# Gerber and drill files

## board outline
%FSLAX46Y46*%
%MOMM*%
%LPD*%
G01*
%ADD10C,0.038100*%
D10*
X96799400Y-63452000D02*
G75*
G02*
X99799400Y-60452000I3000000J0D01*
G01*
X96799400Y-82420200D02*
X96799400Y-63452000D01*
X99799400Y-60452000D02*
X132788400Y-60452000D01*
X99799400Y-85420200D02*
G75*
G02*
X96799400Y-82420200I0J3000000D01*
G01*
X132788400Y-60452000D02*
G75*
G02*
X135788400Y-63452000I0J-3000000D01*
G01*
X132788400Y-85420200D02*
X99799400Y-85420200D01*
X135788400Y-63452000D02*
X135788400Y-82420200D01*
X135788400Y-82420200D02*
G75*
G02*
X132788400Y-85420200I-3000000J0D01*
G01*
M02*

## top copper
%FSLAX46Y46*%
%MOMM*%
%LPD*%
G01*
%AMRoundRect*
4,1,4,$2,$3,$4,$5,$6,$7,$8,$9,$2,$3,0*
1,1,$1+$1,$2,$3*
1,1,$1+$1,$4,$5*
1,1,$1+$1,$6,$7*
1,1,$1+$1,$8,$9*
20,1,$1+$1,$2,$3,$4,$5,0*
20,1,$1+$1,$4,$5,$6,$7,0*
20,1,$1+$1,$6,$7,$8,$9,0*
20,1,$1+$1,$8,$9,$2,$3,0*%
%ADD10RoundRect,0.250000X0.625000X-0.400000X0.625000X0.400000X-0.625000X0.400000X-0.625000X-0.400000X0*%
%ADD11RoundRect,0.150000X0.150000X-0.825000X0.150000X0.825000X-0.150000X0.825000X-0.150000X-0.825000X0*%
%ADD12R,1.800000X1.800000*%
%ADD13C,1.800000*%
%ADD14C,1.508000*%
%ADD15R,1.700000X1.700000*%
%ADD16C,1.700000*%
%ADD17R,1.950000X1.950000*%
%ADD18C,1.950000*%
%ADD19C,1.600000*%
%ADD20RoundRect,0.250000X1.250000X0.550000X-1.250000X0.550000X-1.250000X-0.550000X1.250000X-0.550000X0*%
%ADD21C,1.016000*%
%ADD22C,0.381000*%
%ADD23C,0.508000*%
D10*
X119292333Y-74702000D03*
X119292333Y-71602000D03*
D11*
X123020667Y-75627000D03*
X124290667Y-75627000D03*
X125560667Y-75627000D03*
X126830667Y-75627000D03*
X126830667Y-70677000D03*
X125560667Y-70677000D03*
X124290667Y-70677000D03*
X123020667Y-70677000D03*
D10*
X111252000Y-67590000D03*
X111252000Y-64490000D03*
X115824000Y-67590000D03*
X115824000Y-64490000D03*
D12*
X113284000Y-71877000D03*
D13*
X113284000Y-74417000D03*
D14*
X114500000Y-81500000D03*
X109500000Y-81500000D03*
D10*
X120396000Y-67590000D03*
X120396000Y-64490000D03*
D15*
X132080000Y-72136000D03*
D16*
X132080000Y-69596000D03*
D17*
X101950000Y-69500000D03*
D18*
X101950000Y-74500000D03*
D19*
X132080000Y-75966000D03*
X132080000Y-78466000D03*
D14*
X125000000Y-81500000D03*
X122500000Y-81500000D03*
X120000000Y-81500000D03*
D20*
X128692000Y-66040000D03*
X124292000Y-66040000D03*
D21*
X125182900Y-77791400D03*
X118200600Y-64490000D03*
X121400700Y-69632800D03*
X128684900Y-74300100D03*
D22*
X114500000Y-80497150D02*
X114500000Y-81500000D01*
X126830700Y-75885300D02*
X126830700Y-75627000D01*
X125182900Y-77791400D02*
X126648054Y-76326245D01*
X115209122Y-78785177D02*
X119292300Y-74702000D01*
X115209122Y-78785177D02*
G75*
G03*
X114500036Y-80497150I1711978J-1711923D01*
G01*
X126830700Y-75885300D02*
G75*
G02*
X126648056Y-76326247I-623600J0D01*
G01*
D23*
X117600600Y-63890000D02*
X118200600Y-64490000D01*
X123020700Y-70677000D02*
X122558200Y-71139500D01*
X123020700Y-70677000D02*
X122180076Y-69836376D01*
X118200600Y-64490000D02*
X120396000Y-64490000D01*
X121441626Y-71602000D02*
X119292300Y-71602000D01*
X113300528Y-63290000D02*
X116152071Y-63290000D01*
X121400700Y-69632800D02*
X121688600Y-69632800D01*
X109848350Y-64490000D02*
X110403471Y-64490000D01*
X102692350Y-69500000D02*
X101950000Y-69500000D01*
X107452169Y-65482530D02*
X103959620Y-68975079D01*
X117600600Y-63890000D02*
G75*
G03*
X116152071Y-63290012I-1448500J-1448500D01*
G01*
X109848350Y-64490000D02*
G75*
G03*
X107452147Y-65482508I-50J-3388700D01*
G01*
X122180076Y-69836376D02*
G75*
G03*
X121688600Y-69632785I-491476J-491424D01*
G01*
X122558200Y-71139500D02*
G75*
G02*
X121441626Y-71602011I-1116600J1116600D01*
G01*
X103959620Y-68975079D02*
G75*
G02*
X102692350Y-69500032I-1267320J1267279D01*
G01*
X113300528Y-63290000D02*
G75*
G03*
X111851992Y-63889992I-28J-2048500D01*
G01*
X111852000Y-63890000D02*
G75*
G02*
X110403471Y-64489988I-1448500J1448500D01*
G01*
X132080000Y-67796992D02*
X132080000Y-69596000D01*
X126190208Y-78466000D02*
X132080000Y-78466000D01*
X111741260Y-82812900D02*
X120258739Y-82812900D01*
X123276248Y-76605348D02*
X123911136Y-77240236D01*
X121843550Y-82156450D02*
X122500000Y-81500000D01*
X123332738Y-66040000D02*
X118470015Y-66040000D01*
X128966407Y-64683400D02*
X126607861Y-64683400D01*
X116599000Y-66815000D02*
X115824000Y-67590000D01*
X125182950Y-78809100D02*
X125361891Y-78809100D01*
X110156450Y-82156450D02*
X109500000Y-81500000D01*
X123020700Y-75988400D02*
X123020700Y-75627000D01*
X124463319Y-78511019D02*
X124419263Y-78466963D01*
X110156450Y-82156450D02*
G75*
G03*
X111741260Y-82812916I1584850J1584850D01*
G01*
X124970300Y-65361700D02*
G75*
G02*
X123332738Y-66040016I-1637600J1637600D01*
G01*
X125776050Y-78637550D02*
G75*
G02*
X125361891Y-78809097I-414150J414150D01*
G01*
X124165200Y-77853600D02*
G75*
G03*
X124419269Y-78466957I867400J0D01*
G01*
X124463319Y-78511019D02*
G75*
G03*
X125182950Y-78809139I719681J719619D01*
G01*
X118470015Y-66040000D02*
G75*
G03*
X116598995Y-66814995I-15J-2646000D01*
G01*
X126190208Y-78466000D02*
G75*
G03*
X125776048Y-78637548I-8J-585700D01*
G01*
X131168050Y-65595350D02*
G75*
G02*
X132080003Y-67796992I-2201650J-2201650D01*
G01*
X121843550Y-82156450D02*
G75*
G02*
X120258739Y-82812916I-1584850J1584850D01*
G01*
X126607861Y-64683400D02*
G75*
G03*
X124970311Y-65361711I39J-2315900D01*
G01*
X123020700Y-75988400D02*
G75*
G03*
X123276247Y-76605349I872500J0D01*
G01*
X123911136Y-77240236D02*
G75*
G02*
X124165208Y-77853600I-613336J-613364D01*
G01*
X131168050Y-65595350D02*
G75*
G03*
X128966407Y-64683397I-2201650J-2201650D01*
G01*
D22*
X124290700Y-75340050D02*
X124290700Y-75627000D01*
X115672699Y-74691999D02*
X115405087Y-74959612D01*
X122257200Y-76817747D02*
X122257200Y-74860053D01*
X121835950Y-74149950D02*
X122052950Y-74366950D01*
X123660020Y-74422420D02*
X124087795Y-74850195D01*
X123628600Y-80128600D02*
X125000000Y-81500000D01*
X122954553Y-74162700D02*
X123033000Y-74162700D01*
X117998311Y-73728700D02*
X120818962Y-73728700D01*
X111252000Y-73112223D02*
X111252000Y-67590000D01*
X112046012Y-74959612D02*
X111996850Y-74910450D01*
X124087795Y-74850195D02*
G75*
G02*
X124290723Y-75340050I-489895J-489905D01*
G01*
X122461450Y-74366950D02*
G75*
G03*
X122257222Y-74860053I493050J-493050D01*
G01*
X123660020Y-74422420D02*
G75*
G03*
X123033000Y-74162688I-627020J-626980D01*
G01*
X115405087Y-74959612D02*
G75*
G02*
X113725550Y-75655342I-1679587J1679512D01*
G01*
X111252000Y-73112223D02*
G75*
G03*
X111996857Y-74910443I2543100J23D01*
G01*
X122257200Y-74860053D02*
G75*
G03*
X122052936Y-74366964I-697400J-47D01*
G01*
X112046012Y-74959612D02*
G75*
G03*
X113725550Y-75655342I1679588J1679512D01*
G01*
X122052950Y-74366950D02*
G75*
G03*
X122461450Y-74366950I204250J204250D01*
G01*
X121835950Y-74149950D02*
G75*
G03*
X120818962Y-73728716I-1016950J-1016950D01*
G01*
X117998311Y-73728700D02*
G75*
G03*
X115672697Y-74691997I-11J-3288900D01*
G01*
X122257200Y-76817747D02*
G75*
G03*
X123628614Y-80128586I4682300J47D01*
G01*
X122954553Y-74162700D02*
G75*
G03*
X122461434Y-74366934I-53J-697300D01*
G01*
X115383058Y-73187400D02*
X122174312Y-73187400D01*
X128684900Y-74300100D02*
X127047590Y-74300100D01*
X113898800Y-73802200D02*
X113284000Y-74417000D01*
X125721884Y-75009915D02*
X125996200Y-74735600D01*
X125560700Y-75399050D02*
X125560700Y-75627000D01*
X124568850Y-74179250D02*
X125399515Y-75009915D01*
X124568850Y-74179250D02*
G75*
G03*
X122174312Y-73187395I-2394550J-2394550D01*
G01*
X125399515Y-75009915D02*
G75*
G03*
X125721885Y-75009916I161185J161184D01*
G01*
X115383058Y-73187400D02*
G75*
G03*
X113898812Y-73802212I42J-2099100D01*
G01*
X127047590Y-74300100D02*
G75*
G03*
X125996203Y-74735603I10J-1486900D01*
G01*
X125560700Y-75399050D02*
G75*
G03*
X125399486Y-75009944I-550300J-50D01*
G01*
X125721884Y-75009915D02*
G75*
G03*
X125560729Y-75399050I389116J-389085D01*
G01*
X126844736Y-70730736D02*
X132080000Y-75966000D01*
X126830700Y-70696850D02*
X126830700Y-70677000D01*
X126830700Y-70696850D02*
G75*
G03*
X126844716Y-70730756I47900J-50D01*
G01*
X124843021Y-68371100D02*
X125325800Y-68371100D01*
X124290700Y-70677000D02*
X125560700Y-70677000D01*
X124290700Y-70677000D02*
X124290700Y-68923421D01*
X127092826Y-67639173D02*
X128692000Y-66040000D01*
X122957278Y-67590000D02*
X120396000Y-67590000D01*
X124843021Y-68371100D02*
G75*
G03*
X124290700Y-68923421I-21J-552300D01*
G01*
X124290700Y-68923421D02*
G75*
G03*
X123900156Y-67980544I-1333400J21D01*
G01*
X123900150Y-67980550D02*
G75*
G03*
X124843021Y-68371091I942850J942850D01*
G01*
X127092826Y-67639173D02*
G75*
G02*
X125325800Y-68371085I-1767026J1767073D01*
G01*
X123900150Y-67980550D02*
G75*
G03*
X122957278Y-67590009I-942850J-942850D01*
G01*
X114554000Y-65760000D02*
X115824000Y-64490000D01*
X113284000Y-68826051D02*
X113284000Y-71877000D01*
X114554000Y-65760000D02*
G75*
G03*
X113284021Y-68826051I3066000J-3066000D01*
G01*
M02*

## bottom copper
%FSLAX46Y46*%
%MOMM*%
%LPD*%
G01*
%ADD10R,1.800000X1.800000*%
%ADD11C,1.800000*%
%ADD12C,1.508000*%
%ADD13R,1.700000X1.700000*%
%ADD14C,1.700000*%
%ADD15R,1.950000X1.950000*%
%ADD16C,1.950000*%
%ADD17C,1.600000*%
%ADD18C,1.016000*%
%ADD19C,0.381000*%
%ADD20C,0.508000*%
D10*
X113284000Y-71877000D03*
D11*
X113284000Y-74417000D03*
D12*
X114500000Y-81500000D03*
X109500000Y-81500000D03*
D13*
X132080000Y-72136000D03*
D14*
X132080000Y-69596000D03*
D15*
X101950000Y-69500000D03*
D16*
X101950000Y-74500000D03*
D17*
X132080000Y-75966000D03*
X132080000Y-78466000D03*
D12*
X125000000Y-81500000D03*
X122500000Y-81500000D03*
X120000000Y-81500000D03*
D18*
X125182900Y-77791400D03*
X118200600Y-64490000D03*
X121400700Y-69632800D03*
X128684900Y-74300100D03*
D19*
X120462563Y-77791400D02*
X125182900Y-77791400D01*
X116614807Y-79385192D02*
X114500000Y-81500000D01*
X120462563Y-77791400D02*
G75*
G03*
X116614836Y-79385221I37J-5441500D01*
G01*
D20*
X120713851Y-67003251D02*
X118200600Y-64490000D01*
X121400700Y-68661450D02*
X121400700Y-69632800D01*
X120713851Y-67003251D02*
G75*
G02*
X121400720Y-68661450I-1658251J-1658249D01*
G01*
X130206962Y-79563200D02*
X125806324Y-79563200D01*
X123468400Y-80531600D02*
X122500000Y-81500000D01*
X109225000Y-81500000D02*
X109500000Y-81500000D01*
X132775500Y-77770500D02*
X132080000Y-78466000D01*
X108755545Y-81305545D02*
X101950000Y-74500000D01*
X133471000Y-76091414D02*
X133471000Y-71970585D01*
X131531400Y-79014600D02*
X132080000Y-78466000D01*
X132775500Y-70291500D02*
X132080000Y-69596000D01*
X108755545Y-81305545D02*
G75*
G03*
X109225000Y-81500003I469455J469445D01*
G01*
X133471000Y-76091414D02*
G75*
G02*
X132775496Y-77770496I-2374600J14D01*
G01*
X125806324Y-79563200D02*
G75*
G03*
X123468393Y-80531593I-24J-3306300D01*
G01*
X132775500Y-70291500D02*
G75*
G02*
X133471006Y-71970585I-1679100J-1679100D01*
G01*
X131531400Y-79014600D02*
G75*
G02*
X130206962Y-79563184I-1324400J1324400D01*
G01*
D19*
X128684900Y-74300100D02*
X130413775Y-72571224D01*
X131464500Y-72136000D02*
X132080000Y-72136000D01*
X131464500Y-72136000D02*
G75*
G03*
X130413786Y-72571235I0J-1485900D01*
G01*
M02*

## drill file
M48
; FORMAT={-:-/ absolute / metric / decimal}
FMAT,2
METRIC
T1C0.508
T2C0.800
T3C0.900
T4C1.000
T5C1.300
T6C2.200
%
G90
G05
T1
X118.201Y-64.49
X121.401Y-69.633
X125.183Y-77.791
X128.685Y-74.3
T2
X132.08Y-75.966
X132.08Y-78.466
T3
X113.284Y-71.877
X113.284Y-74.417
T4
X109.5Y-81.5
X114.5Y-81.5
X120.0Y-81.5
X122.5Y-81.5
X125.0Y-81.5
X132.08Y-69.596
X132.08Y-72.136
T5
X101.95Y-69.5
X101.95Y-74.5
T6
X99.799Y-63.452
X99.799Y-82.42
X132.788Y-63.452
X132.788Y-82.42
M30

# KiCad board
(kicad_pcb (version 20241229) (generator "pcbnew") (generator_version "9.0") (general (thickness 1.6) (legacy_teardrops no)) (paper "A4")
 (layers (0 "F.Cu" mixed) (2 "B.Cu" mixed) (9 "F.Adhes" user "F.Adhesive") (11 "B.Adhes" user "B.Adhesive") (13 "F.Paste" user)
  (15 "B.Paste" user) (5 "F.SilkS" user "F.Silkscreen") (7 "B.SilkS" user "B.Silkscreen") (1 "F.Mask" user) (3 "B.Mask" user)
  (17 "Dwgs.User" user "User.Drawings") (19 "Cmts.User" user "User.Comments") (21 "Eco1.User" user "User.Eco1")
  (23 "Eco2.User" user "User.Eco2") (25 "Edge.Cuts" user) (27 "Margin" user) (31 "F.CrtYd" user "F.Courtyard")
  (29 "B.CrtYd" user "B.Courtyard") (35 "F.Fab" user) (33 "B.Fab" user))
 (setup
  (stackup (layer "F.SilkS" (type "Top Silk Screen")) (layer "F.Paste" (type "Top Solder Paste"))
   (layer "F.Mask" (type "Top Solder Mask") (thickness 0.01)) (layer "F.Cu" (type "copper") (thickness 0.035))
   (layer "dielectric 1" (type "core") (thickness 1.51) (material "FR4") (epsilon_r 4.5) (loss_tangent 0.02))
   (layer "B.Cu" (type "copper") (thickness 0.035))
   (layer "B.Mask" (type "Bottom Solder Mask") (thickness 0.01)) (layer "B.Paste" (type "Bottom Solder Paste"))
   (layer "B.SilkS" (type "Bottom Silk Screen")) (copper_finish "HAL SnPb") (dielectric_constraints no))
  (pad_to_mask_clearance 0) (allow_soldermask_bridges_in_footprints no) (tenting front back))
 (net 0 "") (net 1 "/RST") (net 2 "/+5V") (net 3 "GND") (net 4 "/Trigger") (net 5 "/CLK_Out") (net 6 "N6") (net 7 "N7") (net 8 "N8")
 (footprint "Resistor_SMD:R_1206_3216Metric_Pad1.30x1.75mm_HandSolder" (layer "F.Cu") (at 119.292333 73.152 90)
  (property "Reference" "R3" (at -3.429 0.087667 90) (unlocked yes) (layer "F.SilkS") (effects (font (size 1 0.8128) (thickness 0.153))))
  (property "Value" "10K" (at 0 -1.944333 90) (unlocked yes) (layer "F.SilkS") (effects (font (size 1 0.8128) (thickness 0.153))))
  (pad "1" smd roundrect (at -1.55 0 90) (size 1.3 1.75) (layers "F.Cu" "F.Mask" "F.Paste") (roundrect_rratio 0.192308) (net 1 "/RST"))
  (pad "2" smd roundrect (at 1.55 0 90) (size 1.3 1.75) (layers "F.Cu" "F.Mask" "F.Paste") (roundrect_rratio 0.192308) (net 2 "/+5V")))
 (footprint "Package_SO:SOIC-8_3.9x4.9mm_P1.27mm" (layer "F.Cu") (at 124.925667 73.152 90)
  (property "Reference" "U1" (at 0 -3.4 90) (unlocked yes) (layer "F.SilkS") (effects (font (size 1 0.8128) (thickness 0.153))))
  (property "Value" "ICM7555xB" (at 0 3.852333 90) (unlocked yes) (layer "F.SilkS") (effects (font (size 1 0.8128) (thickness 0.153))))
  (pad "1" smd roundrect (at -2.475 -1.905 90) (size 1.95 0.6) (layers "F.Cu" "F.Mask" "F.Paste") (roundrect_rratio 0.25) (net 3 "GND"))
  (pad "2" smd roundrect (at -2.475 -0.635 90) (size 1.95 0.6) (layers "F.Cu" "F.Mask" "F.Paste") (roundrect_rratio 0.25) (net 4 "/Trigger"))
  (pad "3" smd roundrect (at -2.475 0.635 90) (size 1.95 0.6) (layers "F.Cu" "F.Mask" "F.Paste") (roundrect_rratio 0.25) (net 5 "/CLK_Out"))
  (pad "4" smd roundrect (at -2.475 1.905 90) (size 1.95 0.6) (layers "F.Cu" "F.Mask" "F.Paste") (roundrect_rratio 0.25) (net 1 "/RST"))
  (pad "5" smd roundrect (at 2.475 1.905 90) (size 1.95 0.6) (layers "F.Cu" "F.Mask" "F.Paste") (roundrect_rratio 0.25) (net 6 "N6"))
  (pad "6" smd roundrect (at 2.475 0.635 90) (size 1.95 0.6) (layers "F.Cu" "F.Mask" "F.Paste") (roundrect_rratio 0.25) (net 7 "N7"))
  (pad "7" smd roundrect (at 2.475 -0.635 90) (size 1.95 0.6) (layers "F.Cu" "F.Mask" "F.Paste") (roundrect_rratio 0.25) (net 7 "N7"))
  (pad "8" smd roundrect (at 2.475 -1.905 90) (size 1.95 0.6) (layers "F.Cu" "F.Mask" "F.Paste") (roundrect_rratio 0.25) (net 2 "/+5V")))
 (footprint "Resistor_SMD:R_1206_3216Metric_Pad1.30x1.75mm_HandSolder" (layer "F.Cu") (at 111.252 66.04 90)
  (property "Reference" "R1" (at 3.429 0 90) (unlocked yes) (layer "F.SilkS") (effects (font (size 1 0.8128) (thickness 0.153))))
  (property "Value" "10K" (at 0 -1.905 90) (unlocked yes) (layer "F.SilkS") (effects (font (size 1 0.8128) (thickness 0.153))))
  (pad "1" smd roundrect (at -1.55 0 90) (size 1.3 1.75) (layers "F.Cu" "F.Mask" "F.Paste") (roundrect_rratio 0.192308) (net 4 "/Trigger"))
  (pad "2" smd roundrect (at 1.55 0 90) (size 1.3 1.75) (layers "F.Cu" "F.Mask" "F.Paste") (roundrect_rratio 0.192308) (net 2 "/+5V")))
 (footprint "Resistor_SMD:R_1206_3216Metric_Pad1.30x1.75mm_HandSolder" (layer "F.Cu") (at 115.824 66.04 90)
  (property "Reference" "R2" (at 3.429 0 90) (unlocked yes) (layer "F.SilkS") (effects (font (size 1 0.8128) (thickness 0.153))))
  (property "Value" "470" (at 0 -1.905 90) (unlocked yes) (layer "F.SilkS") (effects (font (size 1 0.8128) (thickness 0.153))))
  (pad "1" smd roundrect (at -1.55 0 90) (size 1.3 1.75) (layers "F.Cu" "F.Mask" "F.Paste") (roundrect_rratio 0.192308) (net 3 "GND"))
  (pad "2" smd roundrect (at 1.55 0 90) (size 1.3 1.75) (layers "F.Cu" "F.Mask" "F.Paste") (roundrect_rratio 0.192308) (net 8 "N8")))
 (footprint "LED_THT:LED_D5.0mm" (layer "F.Cu") (at 113.284 71.877 -90)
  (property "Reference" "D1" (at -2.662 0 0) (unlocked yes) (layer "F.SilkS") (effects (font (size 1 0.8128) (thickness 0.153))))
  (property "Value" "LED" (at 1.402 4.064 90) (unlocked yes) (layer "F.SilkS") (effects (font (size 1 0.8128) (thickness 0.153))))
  (pad "1" thru_hole rect (at 0 0 270) (size 1.8 1.8) (drill 0.9) (layers "*.Cu" "*.Mask") (remove_unused_layers no) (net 8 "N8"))
  (pad "2" thru_hole circle (at 2.54 0 270) (size 1.8 1.8) (drill 0.9) (layers "*.Cu" "*.Mask") (remove_unused_layers no) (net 5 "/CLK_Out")))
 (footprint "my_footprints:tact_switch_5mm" (layer "F.Cu") (at 112 81.5 180)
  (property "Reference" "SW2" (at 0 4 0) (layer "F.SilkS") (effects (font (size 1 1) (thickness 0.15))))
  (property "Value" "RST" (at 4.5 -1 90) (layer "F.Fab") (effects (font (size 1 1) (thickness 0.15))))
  (pad "1" thru_hole circle (at -2.5 0 180) (size 1.508 1.508) (drill 1) (layers "*.Cu" "*.Mask") (remove_unused_layers no) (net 1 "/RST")
   (solder_mask_margin 0.102))
  (pad "2" thru_hole circle (at 2.5 0 180) (size 1.508 1.508) (drill 1) (layers "*.Cu" "*.Mask") (remove_unused_layers no) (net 3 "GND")
   (solder_mask_margin 0.102)))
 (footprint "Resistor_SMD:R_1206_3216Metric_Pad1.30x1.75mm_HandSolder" (layer "F.Cu") (at 120.396 66.04 90)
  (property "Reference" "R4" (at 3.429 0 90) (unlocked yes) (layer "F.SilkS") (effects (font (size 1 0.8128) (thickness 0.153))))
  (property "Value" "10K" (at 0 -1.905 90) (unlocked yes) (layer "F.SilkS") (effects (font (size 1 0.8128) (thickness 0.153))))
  (pad "1" smd roundrect (at -1.55 0 90) (size 1.3 1.75) (layers "F.Cu" "F.Mask" "F.Paste") (roundrect_rratio 0.192308) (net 7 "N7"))
  (pad "2" smd roundrect (at 1.55 0 90) (size 1.3 1.75) (layers "F.Cu" "F.Mask" "F.Paste") (roundrect_rratio 0.192308) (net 2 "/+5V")))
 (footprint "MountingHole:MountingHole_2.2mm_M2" (layer "F.Cu") (at 99.7994 63.452)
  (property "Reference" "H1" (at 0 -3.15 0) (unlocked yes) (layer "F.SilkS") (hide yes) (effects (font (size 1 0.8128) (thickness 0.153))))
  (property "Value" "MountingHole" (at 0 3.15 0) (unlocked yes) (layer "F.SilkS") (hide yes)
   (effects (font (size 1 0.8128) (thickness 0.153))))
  (pad "" np_thru_hole circle (at 0 0) (size 2.2 2.2) (drill 2.2) (layers "*.Cu" "*.Mask")))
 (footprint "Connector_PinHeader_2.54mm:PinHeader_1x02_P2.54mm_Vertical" (layer "F.Cu") (at 132.08 72.136 180)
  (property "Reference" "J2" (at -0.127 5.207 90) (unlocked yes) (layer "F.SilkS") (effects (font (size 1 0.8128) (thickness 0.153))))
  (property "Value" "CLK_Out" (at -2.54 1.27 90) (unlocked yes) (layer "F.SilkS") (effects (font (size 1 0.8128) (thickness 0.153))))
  (pad "1" thru_hole rect (at 0 0 180) (size 1.7 1.7) (drill 1) (layers "*.Cu" "*.Mask") (remove_unused_layers no) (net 5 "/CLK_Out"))
  (pad "2" thru_hole circle (at 0 2.54 180) (size 1.7 1.7) (drill 1) (layers "*.Cu" "*.Mask") (remove_unused_layers no) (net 3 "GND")))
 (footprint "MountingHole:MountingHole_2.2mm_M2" (layer "F.Cu") (at 132.7884 82.4202)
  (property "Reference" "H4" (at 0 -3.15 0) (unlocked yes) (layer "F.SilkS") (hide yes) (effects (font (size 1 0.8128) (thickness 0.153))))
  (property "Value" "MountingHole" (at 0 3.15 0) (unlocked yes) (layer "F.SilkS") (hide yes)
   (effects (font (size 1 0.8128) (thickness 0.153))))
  (pad "" np_thru_hole circle (at 0 0) (size 2.2 2.2) (drill 2.2) (layers "*.Cu" "*.Mask")))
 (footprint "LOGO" (layer "F.Cu") (at 105.5 63.5)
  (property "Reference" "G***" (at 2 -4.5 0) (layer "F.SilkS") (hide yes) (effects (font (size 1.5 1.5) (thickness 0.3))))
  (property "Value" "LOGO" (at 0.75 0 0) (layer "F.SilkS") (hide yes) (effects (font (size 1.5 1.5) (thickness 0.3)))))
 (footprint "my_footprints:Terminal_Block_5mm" (layer "F.Cu") (at 101.95 72 -90)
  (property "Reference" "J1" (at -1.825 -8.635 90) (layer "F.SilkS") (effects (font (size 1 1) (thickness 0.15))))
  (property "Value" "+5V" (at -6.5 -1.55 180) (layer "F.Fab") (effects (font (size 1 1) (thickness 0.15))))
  (pad "1" thru_hole rect (at -2.5 0 270) (size 1.95 1.95) (drill 1.3) (layers "*.Cu" "*.Mask") (remove_unused_layers no) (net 2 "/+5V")
   (solder_mask_margin 0.102))
  (pad "2" thru_hole circle (at 2.5 0 270) (size 1.95 1.95) (drill 1.3) (layers "*.Cu" "*.Mask") (remove_unused_layers no) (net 3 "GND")
   (solder_mask_margin 0.102)))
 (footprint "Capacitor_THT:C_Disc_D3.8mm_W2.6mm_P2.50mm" (layer "F.Cu") (at 132.08 75.966 -90)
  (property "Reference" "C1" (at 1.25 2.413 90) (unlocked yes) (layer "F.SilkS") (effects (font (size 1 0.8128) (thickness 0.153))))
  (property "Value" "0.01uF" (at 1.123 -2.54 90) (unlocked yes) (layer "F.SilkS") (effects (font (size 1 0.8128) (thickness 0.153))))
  (pad "1" thru_hole circle (at 0 0 270) (size 1.6 1.6) (drill 0.8) (layers "*.Cu" "*.Mask") (remove_unused_layers no) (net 6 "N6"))
  (pad "2" thru_hole circle (at 2.5 0 270) (size 1.6 1.6) (drill 0.8) (layers "*.Cu" "*.Mask") (remove_unused_layers no) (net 3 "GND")))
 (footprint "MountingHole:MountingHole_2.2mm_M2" (layer "F.Cu") (at 132.7884 63.452)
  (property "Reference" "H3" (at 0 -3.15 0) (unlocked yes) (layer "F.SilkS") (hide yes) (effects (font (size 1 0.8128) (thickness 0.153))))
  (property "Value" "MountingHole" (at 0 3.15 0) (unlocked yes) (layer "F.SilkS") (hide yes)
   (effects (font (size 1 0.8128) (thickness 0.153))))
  (pad "" np_thru_hole circle (at 0 0) (size 2.2 2.2) (drill 2.2) (layers "*.Cu" "*.Mask")))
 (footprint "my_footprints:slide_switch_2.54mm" (layer "F.Cu") (at 122.5 81.5 180)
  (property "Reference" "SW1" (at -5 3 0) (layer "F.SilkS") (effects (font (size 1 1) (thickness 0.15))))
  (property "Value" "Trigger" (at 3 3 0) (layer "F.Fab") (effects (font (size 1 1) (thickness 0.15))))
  (pad "1" thru_hole circle (at -2.5 0 180) (size 1.508 1.508) (drill 1) (layers "*.Cu" "*.Mask") (remove_unused_layers no)
   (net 4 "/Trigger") (solder_mask_margin 0.102))
  (pad "2" thru_hole circle (at 0 0 180) (size 1.508 1.508) (drill 1) (layers "*.Cu" "*.Mask") (remove_unused_layers no) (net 3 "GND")
   (solder_mask_margin 0.102))
  (pad "3" thru_hole circle (at 2.5 0 180) (size 1.508 1.508) (drill 1) (layers "*.Cu" "*.Mask") (remove_unused_layers no)
   (solder_mask_margin 0.102)))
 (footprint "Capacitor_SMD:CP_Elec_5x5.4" (layer "F.Cu") (at 126.492 66.04 180)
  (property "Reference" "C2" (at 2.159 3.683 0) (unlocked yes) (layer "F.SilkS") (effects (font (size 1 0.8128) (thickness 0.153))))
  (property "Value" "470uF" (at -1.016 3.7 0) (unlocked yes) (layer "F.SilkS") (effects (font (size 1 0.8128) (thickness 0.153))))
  (pad "1" smd roundrect (at -2.2 0 180) (size 3 1.6) (layers "F.Cu" "F.Mask" "F.Paste") (roundrect_rratio 0.15625) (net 7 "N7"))
  (pad "2" smd roundrect (at 2.2 0 180) (size 3 1.6) (layers "F.Cu" "F.Mask" "F.Paste") (roundrect_rratio 0.15625) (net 3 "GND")))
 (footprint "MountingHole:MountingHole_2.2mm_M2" (layer "F.Cu") (at 99.7994 82.4202)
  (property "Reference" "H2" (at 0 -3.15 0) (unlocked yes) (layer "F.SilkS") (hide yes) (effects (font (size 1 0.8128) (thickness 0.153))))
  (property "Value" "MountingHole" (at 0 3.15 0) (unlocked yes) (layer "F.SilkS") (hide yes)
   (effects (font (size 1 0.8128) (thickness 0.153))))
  (pad "" np_thru_hole circle (at 0 0) (size 2.2 2.2) (drill 2.2) (layers "*.Cu" "*.Mask")))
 (gr_arc (start 96.7994 63.452) (mid 97.67808 61.33068) (end 99.7994 60.452) (stroke (width 0.0381) (type default)) (layer "Edge.Cuts"))
 (gr_line (start 96.7994 82.4202) (end 96.7994 63.452) (stroke (width 0.0381) (type default)) (layer "Edge.Cuts"))
 (gr_line (start 99.7994 60.452) (end 132.7884 60.452) (stroke (width 0.0381) (type default)) (layer "Edge.Cuts"))
 (gr_arc (start 99.7994 85.4202) (mid 97.67808 84.54152) (end 96.7994 82.4202) (stroke (width 0.0381) (type default)) (layer "Edge.Cuts"))
 (gr_arc (start 132.7884 60.452) (mid 134.90972 61.33068) (end 135.7884 63.452) (stroke (width 0.0381) (type default)) (layer "Edge.Cuts"))
 (gr_line (start 132.7884 85.4202) (end 99.7994 85.4202) (stroke (width 0.0381) (type default)) (layer "Edge.Cuts"))
 (gr_line (start 135.7884 63.452) (end 135.7884 82.4202) (stroke (width 0.0381) (type default)) (layer "Edge.Cuts"))
 (gr_arc (start 135.7884 82.4202) (mid 134.90972 84.54152) (end 132.7884 85.4202) (stroke (width 0.0381) (type default)) (layer "Edge.Cuts"))
 (segment (start 114.500000 80.497150) (end 114.500000 81.500000) (width 0.381000) (layer "F.Cu") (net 1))
 (segment (start 126.830700 75.885300) (end 126.830700 75.627000) (width 0.381000) (layer "F.Cu") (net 1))
 (segment (start 125.182900 77.791400) (end 126.648054 76.326245) (width 0.381000) (layer "F.Cu") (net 1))
 (segment (start 115.209122 78.785177) (end 119.292300 74.702000) (width 0.381000) (layer "F.Cu") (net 1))
 (arc (start 115.209122 78.785177) (mid 114.684294 79.570637) (end 114.500000 80.497150) (width 0.381000) (layer "F.Cu") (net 1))
 (arc (start 126.830700 75.885300) (mid 126.783231 76.123937) (end 126.648054 76.326245) (width 0.381000) (layer "F.Cu") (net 1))
 (segment (start 120.462563 77.791400) (end 125.182900 77.791400) (width 0.381000) (layer "B.Cu") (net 1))
 (segment (start 116.614807 79.385192) (end 114.500000 81.500000) (width 0.381000) (layer "B.Cu") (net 1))
 (arc (start 120.462563 77.791400) (mid 118.380172 78.205613) (end 116.614807 79.385192) (width 0.381000) (layer "B.Cu") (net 1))
 (segment (start 117.600600 63.890000) (end 118.200600 64.490000) (width 0.508000) (layer "F.Cu") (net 2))
 (segment (start 123.020700 70.677000) (end 122.558200 71.139500) (width 0.508000) (layer "F.Cu") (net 2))
 (segment (start 123.020700 70.677000) (end 122.180076 69.836376) (width 0.508000) (layer "F.Cu") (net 2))
 (segment (start 118.200600 64.490000) (end 120.396000 64.490000) (width 0.508000) (layer "F.Cu") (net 2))
 (segment (start 121.441626 71.602000) (end 119.292300 71.602000) (width 0.508000) (layer "F.Cu") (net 2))
 (segment (start 113.300528 63.290000) (end 116.152071 63.290000) (width 0.508000) (layer "F.Cu") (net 2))
 (segment (start 121.400700 69.632800) (end 121.688600 69.632800) (width 0.508000) (layer "F.Cu") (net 2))
 (segment (start 109.848350 64.490000) (end 110.403471 64.490000) (width 0.508000) (layer "F.Cu") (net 2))
 (segment (start 102.692350 69.500000) (end 101.950000 69.500000) (width 0.508000) (layer "F.Cu") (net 2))
 (segment (start 107.452169 65.482530) (end 103.959620 68.975079) (width 0.508000) (layer "F.Cu") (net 2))
 (arc (start 117.600600 63.890000) (mid 116.936009 63.445934) (end 116.152071 63.290000) (width 0.508000) (layer "F.Cu") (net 2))
 (arc (start 109.848350 64.490000) (mid 108.551546 64.747950) (end 107.452169 65.482530) (width 0.508000) (layer "F.Cu") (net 2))
 (arc (start 122.180076 69.836376) (mid 121.954584 69.685707) (end 121.688600 69.632800) (width 0.508000) (layer "F.Cu") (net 2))
 (arc (start 122.558200 71.139500) (mid 122.045911 71.481800) (end 121.441626 71.602000) (width 0.508000) (layer "F.Cu") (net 2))
 (arc (start 103.959620 68.975079) (mid 103.378191 69.363577) (end 102.692350 69.500000) (width 0.508000) (layer "F.Cu") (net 2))
 (arc (start 113.300528 63.290000) (mid 112.516590 63.445934) (end 111.852000 63.890000) (width 0.508000) (layer "F.Cu") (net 2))
 (arc (start 111.852000 63.890000) (mid 111.187409 64.334065) (end 110.403471 64.490000) (width 0.508000) (layer "F.Cu") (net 2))
 (segment (start 120.713851 67.003251) (end 118.200600 64.490000) (width 0.508000) (layer "B.Cu") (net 2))
 (segment (start 121.400700 68.661450) (end 121.400700 69.632800) (width 0.508000) (layer "B.Cu") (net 2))
 (arc (start 120.713851 67.003251) (mid 121.222193 67.764039) (end 121.400700 68.661450) (width 0.508000) (layer "B.Cu") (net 2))
 (segment (start 132.080000 67.796992) (end 132.080000 69.596000) (width 0.508000) (layer "F.Cu") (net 3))
 (segment (start 126.190208 78.466000) (end 132.080000 78.466000) (width 0.508000) (layer "F.Cu") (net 3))
 (segment (start 111.741260 82.812900) (end 120.258739 82.812900) (width 0.508000) (layer "F.Cu") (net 3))
 (segment (start 123.276248 76.605348) (end 123.911136 77.240236) (width 0.508000) (layer "F.Cu") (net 3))
 (segment (start 121.843550 82.156450) (end 122.500000 81.500000) (width 0.508000) (layer "F.Cu") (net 3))
 (segment (start 123.332738 66.040000) (end 118.470015 66.040000) (width 0.508000) (layer "F.Cu") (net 3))
 (segment (start 128.966407 64.683400) (end 126.607861 64.683400) (width 0.508000) (layer "F.Cu") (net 3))
 (segment (start 116.599000 66.815000) (end 115.824000 67.590000) (width 0.508000) (layer "F.Cu") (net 3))
 (segment (start 125.182950 78.809100) (end 125.361891 78.809100) (width 0.508000) (layer "F.Cu") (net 3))
 (segment (start 110.156450 82.156450) (end 109.500000 81.500000) (width 0.508000) (layer "F.Cu") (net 3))
 (segment (start 123.020700 75.988400) (end 123.020700 75.627000) (width 0.508000) (layer "F.Cu") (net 3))
 (segment (start 124.463319 78.511019) (end 124.419263 78.466963) (width 0.508000) (layer "F.Cu") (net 3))
 (arc (start 110.156450 82.156450) (mid 110.883567 82.642294) (end 111.741260 82.812900) (width 0.508000) (layer "F.Cu") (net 3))
 (arc (start 124.970300 65.361700) (mid 124.218980 65.863715) (end 123.332738 66.040000) (width 0.508000) (layer "F.Cu") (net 3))
 (arc (start 125.776050 78.637550) (mid 125.586032 78.764515) (end 125.361891 78.809100) (width 0.508000) (layer "F.Cu") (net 3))
 (arc (start 124.165200 77.853600) (mid 124.231228 78.185549) (end 124.419263 78.466963) (width 0.508000) (layer "F.Cu") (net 3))
 (arc (start 124.463319 78.511019) (mid 124.793488 78.731631) (end 125.182950 78.809100) (width 0.508000) (layer "F.Cu") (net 3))
 (arc (start 118.470015 66.040000) (mid 117.457429 66.241415) (end 116.599000 66.815000) (width 0.508000) (layer "F.Cu") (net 3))
 (arc (start 126.190208 78.466000) (mid 125.966067 78.510584) (end 125.776050 78.637550) (width 0.508000) (layer "F.Cu") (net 3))
 (arc (start 131.168050 65.595350) (mid 131.842991 66.605471) (end 132.080000 67.796992) (width 0.508000) (layer "F.Cu") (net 3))
 (arc (start 121.843550 82.156450) (mid 121.116432 82.642294) (end 120.258739 82.812900) (width 0.508000) (layer "F.Cu") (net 3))
 (arc (start 126.607861 64.683400) (mid 125.721619 64.859684) (end 124.970300 65.361700) (width 0.508000) (layer "F.Cu") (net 3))
 (arc (start 123.020700 75.988400) (mid 123.087114 76.322289) (end 123.276248 76.605348) (width 0.508000) (layer "F.Cu") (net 3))
 (arc (start 123.911136 77.240236) (mid 124.099170 77.521649) (end 124.165200 77.853600) (width 0.508000) (layer "F.Cu") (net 3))
 (arc (start 131.168050 65.595350) (mid 130.157927 64.920408) (end 128.966407 64.683400) (width 0.508000) (layer "F.Cu") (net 3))
 (segment (start 130.206962 79.563200) (end 125.806324 79.563200) (width 0.508000) (layer "B.Cu") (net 3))
 (segment (start 123.468400 80.531600) (end 122.500000 81.500000) (width 0.508000) (layer "B.Cu") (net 3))
 (segment (start 109.225000 81.500000) (end 109.500000 81.500000) (width 0.508000) (layer "B.Cu") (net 3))
 (segment (start 132.775500 77.770500) (end 132.080000 78.466000) (width 0.508000) (layer "B.Cu") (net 3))
 (segment (start 108.755545 81.305545) (end 101.950000 74.500000) (width 0.508000) (layer "B.Cu") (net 3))
 (segment (start 133.471000 76.091414) (end 133.471000 71.970585) (width 0.508000) (layer "B.Cu") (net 3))
 (segment (start 131.531400 79.014600) (end 132.080000 78.466000) (width 0.508000) (layer "B.Cu") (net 3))
 (segment (start 132.775500 70.291500) (end 132.080000 69.596000) (width 0.508000) (layer "B.Cu") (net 3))
 (arc (start 108.755545 81.305545) (mid 108.970932 81.449462) (end 109.225000 81.500000) (width 0.508000) (layer "B.Cu") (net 3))
 (arc (start 133.471000 76.091414) (mid 133.290245 77.000128) (end 132.775500 77.770500) (width 0.508000) (layer "B.Cu") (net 3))
 (arc (start 125.806324 79.563200) (mid 124.541048 79.814878) (end 123.468400 80.531600) (width 0.508000) (layer "B.Cu") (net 3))
 (arc (start 132.775500 70.291500) (mid 133.290245 71.061870) (end 133.471000 71.970585) (width 0.508000) (layer "B.Cu") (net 3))
 (arc (start 131.531400 79.014600) (mid 130.923742 79.420623) (end 130.206962 79.563200) (width 0.508000) (layer "B.Cu") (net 3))
 (segment (start 124.290700 75.340050) (end 124.290700 75.627000) (width 0.381000) (layer "F.Cu") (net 4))
 (segment (start 115.672699 74.691999) (end 115.405087 74.959612) (width 0.381000) (layer "F.Cu") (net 4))
 (segment (start 122.257200 76.817747) (end 122.257200 74.860053) (width 0.381000) (layer "F.Cu") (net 4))
 (segment (start 121.835950 74.149950) (end 122.052950 74.366950) (width 0.381000) (layer "F.Cu") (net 4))
 (segment (start 123.660020 74.422420) (end 124.087795 74.850195) (width 0.381000) (layer "F.Cu") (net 4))
 (segment (start 123.628600 80.128600) (end 125.000000 81.500000) (width 0.381000) (layer "F.Cu") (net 4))
 (segment (start 122.954553 74.162700) (end 123.033000 74.162700) (width 0.381000) (layer "F.Cu") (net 4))
 (segment (start 117.998311 73.728700) (end 120.818962 73.728700) (width 0.381000) (layer "F.Cu") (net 4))
 (segment (start 111.252000 73.112223) (end 111.252000 67.590000) (width 0.381000) (layer "F.Cu") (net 4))
 (segment (start 112.046012 74.959612) (end 111.996850 74.910450) (width 0.381000) (layer "F.Cu") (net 4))
 (arc (start 124.087795 74.850195) (mid 124.237966 75.074942) (end 124.290700 75.340050) (width 0.381000) (layer "F.Cu") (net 4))
 (arc (start 122.461450 74.366950) (mid 122.310282 74.593187) (end 122.257200 74.860053) (width 0.381000) (layer "F.Cu") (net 4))
 (arc (start 123.660020 74.422420) (mid 123.372340 74.230199) (end 123.033000 74.162700) (width 0.381000) (layer "F.Cu") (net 4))
 (arc (start 115.405087 74.959612) (mid 114.634508 75.474496) (end 113.725550 75.655300) (width 0.381000) (layer "F.Cu") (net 4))
 (arc (start 111.252000 73.112223) (mid 111.445580 74.085416) (end 111.996850 74.910450) (width 0.381000) (layer "F.Cu") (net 4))
 (arc (start 122.257200 74.860053) (mid 122.204117 74.593187) (end 122.052950 74.366950) (width 0.381000) (layer "F.Cu") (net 4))
 (arc (start 112.046012 74.959612) (mid 112.816590 75.474496) (end 113.725550 75.655300) (width 0.381000) (layer "F.Cu") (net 4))
 (arc (start 122.052950 74.366950) (mid 122.257200 74.451553) (end 122.461450 74.366950) (width 0.381000) (layer "F.Cu") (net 4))
 (arc (start 121.835950 74.149950) (mid 121.369352 73.838179) (end 120.818962 73.728700) (width 0.381000) (layer "F.Cu") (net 4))
 (arc (start 117.998311 73.728700) (mid 116.739699 73.979053) (end 115.672699 74.691999) (width 0.381000) (layer "F.Cu") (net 4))
 (arc (start 122.257200 76.817747) (mid 122.613615 78.609567) (end 123.628600 80.128600) (width 0.381000) (layer "F.Cu") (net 4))
 (arc (start 122.954553 74.162700) (mid 122.687687 74.215782) (end 122.461450 74.366950) (width 0.381000) (layer "F.Cu") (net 4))
 (segment (start 115.383058 73.187400) (end 122.174312 73.187400) (width 0.381000) (layer "F.Cu") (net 5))
 (segment (start 128.684900 74.300100) (end 127.047590 74.300100) (width 0.381000) (layer "F.Cu") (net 5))
 (segment (start 113.898800 73.802200) (end 113.284000 74.417000) (width 0.381000) (layer "F.Cu") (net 5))
 (segment (start 125.721884 75.009915) (end 125.996200 74.735600) (width 0.381000) (layer "F.Cu") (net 5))
 (segment (start 125.560700 75.399050) (end 125.560700 75.627000) (width 0.381000) (layer "F.Cu") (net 5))
 (segment (start 124.568850 74.179250) (end 125.399515 75.009915) (width 0.381000) (layer "F.Cu") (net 5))
 (arc (start 124.568850 74.179250) (mid 123.470226 73.445173) (end 122.174312 73.187400) (width 0.381000) (layer "F.Cu") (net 5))
 (arc (start 125.399515 75.009915) (mid 125.560699 75.076680) (end 125.721884 75.009915) (width 0.381000) (layer "F.Cu") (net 5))
 (arc (start 115.383058 73.187400) (mid 114.579783 73.347181) (end 113.898800 73.802200) (width 0.381000) (layer "F.Cu") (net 5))
 (arc (start 127.047590 74.300100) (mid 126.478581 74.413282) (end 125.996200 74.735600) (width 0.381000) (layer "F.Cu") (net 5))
 (arc (start 125.560700 75.399050) (mid 125.518809 75.188451) (end 125.399515 75.009915) (width 0.381000) (layer "F.Cu") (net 5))
 (arc (start 125.721884 75.009915) (mid 125.602590 75.188451) (end 125.560700 75.399050) (width 0.381000) (layer "F.Cu") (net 5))
 (segment (start 128.684900 74.300100) (end 130.413775 72.571224) (width 0.381000) (layer "B.Cu") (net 5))
 (segment (start 131.464500 72.136000) (end 132.080000 72.136000) (width 0.381000) (layer "B.Cu") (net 5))
 (arc (start 131.464500 72.136000) (mid 130.895851 72.249111) (end 130.413775 72.571224) (width 0.381000) (layer "B.Cu") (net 5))
 (segment (start 126.844736 70.730736) (end 132.080000 75.966000) (width 0.381000) (layer "F.Cu") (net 6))
 (segment (start 126.830700 70.696850) (end 126.830700 70.677000) (width 0.381000) (layer "F.Cu") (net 6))
 (arc (start 126.830700 70.696850) (mid 126.834347 70.715188) (end 126.844736 70.730736) (width 0.381000) (layer "F.Cu") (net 6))
 (segment (start 124.843021 68.371100) (end 125.325800 68.371100) (width 0.381000) (layer "F.Cu") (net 7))
 (segment (start 124.290700 70.677000) (end 125.560700 70.677000) (width 0.381000) (layer "F.Cu") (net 7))
 (segment (start 124.290700 70.677000) (end 124.290700 68.923421) (width 0.381000) (layer "F.Cu") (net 7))
 (segment (start 127.092826 67.639173) (end 128.692000 66.040000) (width 0.381000) (layer "F.Cu") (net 7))
 (segment (start 122.957278 67.590000) (end 120.396000 67.590000) (width 0.381000) (layer "F.Cu") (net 7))
 (arc (start 124.843021 68.371100) (mid 124.452471 68.532871) (end 124.290700 68.923421) (width 0.381000) (layer "F.Cu") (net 7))
 (arc (start 124.290700 68.923421) (mid 124.189199 68.413142) (end 123.900150 67.980550) (width 0.381000) (layer "F.Cu") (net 7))
 (arc (start 123.900150 67.980550) (mid 124.332742 68.269599) (end 124.843021 68.371100) (width 0.381000) (layer "F.Cu") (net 7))
 (arc (start 127.092826 67.639173) (mid 126.282107 68.180878) (end 125.325800 68.371100) (width 0.381000) (layer "F.Cu") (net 7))
 (arc (start 123.900150 67.980550) (mid 123.467556 67.691500) (end 122.957278 67.590000) (width 0.381000) (layer "F.Cu") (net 7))
 (segment (start 114.554000 65.760000) (end 115.824000 64.490000) (width 0.381000) (layer "F.Cu") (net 8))
 (segment (start 113.284000 68.826051) (end 113.284000 71.877000) (width 0.381000) (layer "F.Cu") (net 8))
 (arc (start 114.554000 65.760000) (mid 113.614062 67.166716) (end 113.284000 68.826051) (width 0.381000) (layer "F.Cu") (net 8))
 (via (at 125.182900 77.791400) (size 1.016000) (drill 0.508000) (layers "F.Cu" "B.Cu") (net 1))
 (via (at 118.200600 64.490000) (size 1.016000) (drill 0.508000) (layers "F.Cu" "B.Cu") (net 2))
 (via (at 121.400700 69.632800) (size 1.016000) (drill 0.508000) (layers "F.Cu" "B.Cu") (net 2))
 (via (at 128.684900 74.300100) (size 1.016000) (drill 0.508000) (layers "F.Cu" "B.Cu") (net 5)))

